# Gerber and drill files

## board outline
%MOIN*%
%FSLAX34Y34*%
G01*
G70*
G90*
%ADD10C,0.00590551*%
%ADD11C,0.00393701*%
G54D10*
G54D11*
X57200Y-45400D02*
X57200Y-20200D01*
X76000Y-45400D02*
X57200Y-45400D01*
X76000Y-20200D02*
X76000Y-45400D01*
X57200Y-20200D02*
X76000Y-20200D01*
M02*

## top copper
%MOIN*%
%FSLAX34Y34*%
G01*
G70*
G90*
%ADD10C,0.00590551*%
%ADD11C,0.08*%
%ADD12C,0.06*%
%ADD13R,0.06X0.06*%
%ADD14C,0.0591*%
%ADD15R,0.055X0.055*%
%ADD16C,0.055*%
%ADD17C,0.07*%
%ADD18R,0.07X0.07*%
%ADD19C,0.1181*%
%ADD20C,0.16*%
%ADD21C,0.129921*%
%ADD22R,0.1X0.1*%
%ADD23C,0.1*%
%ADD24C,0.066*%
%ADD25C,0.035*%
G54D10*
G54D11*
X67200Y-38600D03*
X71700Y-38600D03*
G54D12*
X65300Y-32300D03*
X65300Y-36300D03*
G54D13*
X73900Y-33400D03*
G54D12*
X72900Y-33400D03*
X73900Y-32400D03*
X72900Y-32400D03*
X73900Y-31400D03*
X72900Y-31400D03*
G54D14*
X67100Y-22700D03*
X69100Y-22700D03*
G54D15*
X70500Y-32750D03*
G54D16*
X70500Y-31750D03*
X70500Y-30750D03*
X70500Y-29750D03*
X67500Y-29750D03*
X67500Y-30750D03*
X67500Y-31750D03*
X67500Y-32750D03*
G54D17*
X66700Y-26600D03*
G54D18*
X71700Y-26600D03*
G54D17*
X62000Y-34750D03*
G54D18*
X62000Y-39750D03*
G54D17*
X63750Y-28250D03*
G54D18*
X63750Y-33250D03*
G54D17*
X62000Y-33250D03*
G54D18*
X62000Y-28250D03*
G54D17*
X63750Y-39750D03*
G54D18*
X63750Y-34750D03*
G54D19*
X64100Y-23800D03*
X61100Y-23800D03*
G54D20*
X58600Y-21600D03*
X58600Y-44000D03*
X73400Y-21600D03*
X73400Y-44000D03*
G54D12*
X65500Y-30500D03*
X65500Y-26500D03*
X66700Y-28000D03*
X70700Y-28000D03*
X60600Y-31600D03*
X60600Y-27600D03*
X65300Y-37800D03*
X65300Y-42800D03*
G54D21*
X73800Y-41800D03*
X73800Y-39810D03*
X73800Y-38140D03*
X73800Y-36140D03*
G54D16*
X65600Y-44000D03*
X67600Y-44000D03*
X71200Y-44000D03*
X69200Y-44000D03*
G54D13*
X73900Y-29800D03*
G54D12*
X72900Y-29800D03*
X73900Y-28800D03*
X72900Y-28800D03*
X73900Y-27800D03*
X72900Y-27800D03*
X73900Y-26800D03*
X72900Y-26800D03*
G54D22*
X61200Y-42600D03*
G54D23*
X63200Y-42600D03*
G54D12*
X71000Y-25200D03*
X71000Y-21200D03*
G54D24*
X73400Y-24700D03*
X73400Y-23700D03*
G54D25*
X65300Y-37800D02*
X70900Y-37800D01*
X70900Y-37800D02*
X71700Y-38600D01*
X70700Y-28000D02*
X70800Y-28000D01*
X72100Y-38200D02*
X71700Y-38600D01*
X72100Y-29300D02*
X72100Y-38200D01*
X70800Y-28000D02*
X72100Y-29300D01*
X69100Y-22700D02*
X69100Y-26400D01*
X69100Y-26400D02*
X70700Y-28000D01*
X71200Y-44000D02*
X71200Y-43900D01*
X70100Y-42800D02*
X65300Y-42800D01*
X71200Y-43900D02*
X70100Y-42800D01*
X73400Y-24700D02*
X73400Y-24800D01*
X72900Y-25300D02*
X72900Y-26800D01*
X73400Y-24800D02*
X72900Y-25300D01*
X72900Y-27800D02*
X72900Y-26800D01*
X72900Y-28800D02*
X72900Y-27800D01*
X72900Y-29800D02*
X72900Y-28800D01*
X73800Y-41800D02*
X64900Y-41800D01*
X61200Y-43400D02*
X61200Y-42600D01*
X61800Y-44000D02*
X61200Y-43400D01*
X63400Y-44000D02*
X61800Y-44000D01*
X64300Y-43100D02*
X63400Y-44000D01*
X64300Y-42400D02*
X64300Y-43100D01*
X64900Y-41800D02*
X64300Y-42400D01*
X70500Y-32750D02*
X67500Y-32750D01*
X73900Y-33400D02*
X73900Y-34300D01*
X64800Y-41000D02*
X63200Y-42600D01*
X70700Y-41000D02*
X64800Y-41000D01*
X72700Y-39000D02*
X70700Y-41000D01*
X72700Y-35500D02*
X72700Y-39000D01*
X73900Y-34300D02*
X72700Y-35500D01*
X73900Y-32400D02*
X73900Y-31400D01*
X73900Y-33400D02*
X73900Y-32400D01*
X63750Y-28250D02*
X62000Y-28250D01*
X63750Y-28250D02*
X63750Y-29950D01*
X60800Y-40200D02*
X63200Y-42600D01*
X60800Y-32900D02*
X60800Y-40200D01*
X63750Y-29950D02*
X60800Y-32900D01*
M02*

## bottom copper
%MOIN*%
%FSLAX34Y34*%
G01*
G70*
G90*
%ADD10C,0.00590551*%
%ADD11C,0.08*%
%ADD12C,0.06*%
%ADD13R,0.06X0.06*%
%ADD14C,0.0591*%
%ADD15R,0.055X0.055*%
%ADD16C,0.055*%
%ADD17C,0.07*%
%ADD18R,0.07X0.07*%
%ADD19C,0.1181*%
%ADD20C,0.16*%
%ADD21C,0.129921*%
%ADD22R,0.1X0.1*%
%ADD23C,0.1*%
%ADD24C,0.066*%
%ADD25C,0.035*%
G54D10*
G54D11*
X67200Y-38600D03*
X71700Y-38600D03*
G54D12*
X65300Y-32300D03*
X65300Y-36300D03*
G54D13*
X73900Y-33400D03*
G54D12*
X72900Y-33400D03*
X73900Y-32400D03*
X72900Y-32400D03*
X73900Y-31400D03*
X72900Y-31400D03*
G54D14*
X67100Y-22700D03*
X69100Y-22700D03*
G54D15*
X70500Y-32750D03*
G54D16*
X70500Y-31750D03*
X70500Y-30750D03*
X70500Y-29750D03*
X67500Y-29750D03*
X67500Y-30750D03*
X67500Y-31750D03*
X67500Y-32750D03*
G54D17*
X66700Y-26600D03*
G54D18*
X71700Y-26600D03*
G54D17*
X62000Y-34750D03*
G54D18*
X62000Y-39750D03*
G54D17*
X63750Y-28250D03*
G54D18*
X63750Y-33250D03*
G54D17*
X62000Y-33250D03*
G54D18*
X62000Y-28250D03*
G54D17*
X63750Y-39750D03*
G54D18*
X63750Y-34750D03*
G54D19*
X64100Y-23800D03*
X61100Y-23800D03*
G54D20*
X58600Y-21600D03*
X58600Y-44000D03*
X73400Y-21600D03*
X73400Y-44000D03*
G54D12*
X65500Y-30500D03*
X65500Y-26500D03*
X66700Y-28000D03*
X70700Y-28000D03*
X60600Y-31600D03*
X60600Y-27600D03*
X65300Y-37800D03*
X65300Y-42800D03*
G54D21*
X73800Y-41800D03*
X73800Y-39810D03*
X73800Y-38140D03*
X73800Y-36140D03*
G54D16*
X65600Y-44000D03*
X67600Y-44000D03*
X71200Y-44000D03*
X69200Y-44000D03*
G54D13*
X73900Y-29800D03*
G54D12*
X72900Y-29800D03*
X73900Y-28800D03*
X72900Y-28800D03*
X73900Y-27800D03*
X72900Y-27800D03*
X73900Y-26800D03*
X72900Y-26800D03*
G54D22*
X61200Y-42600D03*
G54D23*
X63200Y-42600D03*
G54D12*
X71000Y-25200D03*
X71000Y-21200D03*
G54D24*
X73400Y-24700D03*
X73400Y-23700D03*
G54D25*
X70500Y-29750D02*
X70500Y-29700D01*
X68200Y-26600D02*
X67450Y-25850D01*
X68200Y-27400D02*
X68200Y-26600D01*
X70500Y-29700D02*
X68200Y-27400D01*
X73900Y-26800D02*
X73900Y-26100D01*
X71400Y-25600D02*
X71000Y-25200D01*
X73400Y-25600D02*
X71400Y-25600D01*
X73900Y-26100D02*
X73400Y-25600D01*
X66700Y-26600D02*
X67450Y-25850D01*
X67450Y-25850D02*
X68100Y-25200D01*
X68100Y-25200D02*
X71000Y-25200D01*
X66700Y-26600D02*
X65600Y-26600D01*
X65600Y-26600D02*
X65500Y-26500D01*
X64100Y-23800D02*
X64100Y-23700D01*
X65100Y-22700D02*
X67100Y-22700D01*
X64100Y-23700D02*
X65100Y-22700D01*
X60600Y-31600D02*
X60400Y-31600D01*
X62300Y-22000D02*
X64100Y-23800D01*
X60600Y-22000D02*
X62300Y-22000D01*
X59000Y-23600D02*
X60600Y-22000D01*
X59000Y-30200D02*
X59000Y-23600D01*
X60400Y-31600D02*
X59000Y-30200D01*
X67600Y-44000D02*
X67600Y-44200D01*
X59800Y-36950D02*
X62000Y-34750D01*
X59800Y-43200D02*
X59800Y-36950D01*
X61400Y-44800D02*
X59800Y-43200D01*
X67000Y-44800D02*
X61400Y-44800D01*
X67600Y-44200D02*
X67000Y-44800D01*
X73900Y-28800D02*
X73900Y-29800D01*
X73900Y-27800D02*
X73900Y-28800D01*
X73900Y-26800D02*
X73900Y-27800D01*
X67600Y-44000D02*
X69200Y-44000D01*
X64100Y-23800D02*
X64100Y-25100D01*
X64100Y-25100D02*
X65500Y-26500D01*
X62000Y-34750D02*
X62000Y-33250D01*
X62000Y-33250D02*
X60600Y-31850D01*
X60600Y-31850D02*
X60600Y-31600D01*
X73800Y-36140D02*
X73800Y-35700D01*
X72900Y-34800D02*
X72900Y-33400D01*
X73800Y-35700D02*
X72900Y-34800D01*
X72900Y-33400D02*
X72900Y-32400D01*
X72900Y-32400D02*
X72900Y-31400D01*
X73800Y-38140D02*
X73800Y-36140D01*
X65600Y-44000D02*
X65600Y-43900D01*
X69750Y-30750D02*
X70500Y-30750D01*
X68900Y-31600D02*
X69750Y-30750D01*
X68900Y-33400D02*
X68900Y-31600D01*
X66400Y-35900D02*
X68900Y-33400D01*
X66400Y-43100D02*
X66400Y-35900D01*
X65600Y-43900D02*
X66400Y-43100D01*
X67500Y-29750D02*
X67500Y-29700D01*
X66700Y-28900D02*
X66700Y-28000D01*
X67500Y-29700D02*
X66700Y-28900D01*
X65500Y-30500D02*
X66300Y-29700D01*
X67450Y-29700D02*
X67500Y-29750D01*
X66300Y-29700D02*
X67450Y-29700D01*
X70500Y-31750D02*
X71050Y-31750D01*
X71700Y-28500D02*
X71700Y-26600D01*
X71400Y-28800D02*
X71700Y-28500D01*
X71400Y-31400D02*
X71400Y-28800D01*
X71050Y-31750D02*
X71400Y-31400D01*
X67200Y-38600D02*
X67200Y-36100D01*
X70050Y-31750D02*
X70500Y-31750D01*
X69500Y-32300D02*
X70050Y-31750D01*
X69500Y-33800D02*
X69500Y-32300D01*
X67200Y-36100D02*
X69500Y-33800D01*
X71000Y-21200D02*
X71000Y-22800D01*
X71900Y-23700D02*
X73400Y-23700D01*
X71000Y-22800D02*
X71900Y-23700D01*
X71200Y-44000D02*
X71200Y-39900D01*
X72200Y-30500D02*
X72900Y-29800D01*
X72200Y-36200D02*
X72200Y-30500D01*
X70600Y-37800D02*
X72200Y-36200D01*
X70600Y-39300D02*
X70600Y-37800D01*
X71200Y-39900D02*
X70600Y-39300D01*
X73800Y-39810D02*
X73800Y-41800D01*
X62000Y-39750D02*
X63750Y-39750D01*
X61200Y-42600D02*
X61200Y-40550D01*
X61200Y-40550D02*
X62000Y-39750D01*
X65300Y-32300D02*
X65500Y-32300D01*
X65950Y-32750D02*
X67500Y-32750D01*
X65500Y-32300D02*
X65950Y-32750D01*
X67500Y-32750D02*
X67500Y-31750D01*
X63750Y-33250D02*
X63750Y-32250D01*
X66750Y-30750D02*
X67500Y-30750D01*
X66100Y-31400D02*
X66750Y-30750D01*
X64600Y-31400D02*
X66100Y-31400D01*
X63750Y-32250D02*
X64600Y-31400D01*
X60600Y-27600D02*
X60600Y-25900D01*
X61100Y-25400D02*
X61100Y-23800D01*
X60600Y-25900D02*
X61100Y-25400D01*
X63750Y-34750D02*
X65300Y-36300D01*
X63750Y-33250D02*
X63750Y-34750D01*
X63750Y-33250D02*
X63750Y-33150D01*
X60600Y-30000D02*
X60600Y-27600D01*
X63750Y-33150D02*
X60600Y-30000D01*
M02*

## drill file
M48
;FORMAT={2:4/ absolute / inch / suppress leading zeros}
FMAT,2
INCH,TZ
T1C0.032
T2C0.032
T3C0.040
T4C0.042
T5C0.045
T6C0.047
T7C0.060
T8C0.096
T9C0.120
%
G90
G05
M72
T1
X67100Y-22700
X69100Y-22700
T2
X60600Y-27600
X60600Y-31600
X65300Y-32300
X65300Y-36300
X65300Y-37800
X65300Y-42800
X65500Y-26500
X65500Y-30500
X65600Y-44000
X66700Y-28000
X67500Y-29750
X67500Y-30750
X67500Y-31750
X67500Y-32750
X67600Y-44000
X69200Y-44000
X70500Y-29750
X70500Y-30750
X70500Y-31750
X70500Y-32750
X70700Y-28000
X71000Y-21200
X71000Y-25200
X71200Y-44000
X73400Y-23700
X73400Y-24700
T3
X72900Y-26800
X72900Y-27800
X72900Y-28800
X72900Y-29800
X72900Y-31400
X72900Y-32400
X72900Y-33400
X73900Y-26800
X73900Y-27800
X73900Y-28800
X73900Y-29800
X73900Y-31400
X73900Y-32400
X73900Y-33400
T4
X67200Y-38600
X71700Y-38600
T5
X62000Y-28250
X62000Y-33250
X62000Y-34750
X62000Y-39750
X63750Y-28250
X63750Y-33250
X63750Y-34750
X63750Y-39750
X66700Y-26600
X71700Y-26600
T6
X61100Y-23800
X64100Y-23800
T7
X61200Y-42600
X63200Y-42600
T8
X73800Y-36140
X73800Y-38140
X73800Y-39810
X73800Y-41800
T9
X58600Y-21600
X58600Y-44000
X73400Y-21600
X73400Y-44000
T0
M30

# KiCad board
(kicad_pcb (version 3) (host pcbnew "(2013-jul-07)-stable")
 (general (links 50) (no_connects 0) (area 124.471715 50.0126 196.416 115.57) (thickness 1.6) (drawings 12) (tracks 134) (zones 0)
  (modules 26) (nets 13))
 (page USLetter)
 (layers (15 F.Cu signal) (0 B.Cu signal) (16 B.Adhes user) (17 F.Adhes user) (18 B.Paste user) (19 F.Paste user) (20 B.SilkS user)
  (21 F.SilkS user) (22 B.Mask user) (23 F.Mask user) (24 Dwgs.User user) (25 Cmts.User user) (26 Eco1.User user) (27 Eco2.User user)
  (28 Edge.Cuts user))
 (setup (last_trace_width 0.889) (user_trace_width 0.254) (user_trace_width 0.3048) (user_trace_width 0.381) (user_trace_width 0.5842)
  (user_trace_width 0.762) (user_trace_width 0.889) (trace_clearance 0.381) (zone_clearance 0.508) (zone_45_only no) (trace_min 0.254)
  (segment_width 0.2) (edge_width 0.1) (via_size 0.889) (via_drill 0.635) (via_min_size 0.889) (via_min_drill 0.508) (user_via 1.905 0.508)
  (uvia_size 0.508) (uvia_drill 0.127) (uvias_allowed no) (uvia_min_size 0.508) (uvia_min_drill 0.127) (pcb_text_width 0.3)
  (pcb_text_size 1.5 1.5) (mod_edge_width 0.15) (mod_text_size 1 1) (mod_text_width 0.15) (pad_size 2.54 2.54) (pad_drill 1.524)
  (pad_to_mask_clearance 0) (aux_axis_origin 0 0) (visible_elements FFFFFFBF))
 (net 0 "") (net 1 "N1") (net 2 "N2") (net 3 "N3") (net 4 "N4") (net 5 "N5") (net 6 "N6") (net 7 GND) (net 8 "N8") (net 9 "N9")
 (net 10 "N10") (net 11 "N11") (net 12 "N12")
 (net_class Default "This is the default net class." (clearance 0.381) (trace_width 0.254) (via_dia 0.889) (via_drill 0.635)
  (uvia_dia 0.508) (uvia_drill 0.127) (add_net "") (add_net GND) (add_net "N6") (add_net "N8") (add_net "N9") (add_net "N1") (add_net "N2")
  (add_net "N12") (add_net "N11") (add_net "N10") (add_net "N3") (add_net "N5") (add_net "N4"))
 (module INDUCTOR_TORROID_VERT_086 (layer F.Cu) (at 176.276 98.044 90)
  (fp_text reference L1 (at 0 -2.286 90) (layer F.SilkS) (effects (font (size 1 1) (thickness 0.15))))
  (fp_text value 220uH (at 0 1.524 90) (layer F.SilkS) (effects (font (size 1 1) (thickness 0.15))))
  (pad 1 thru_hole circle (at 0 -5.588 90) (size 2.032 2.032) (drill 1.0668) (layers *.Cu *.Mask F.SilkS) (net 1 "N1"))
  (pad 2 thru_hole circle (at 0 5.842 90) (size 2.032 2.032) (drill 1.0668) (layers *.Cu *.Mask F.SilkS) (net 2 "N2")))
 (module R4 (layer F.Cu) (at 165.862 87.122 270) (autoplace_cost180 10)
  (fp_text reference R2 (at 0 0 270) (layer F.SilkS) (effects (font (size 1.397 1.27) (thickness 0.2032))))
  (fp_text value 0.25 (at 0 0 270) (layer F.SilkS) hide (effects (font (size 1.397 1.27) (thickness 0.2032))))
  (pad 1 thru_hole circle (at -5.08 0 270) (size 1.524 1.524) (drill 0.8128) (layers *.Cu *.Mask F.SilkS) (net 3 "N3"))
  (pad 2 thru_hole circle (at 5.08 0 270) (size 1.524 1.524) (drill 0.8128) (layers *.Cu *.Mask F.SilkS) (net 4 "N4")))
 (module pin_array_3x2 (layer F.Cu) (at 186.436 82.296 90)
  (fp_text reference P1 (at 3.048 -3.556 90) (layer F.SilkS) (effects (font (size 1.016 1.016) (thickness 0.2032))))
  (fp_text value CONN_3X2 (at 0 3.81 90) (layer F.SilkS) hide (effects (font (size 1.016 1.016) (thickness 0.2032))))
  (pad 1 thru_hole rect (at -2.54 1.27 90) (size 1.524 1.524) (drill 1.016) (layers *.Cu *.Mask F.SilkS) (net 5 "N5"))
  (pad 2 thru_hole circle (at -2.54 -1.27 90) (size 1.524 1.524) (drill 1.016) (layers *.Cu *.Mask F.SilkS) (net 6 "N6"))
  (pad 3 thru_hole circle (at 0 1.27 90) (size 1.524 1.524) (drill 1.016) (layers *.Cu *.Mask F.SilkS) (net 5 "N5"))
  (pad 4 thru_hole circle (at 0 -1.27 90) (size 1.524 1.524) (drill 1.016) (layers *.Cu *.Mask F.SilkS) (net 6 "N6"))
  (pad 5 thru_hole circle (at 2.54 1.27 90) (size 1.524 1.524) (drill 1.016) (layers *.Cu *.Mask F.SilkS) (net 5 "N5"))
  (pad 6 thru_hole circle (at 2.54 -1.27 90) (size 1.524 1.524) (drill 1.016) (layers *.Cu *.Mask F.SilkS) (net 6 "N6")))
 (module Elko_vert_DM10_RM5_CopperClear (layer F.Cu) (at 172.974 57.658 180)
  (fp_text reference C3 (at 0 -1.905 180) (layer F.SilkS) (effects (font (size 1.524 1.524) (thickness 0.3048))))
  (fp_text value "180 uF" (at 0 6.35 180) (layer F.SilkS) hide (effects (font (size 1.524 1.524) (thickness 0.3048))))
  (pad 2 thru_hole circle (at 2.54 0 180) (size 1.50114 1.50114) (drill 0.8001) (layers *.Cu *.Mask F.SilkS) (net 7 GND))
  (pad 1 thru_hole circle (at -2.54 0 180) (size 1.50114 1.50114) (drill 0.8001) (layers *.Cu *.Mask F.SilkS) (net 2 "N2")))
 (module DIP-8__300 (layer F.Cu) (at 175.26 79.375 90)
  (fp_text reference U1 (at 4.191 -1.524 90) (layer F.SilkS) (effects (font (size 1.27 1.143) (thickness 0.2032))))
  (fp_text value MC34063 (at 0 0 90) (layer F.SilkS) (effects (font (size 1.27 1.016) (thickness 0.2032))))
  (pad 1 thru_hole rect (at -3.81 3.81 90) (size 1.397 1.397) (drill 0.8128) (layers *.Cu *.Mask F.SilkS) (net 3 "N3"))
  (pad 2 thru_hole circle (at -1.27 3.81 90) (size 1.397 1.397) (drill 0.8128) (layers *.Cu *.Mask F.SilkS) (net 1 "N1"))
  (pad 3 thru_hole circle (at 1.27 3.81 90) (size 1.397 1.397) (drill 0.8128) (layers *.Cu *.Mask F.SilkS) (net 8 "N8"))
  (pad 4 thru_hole circle (at 3.81 3.81 90) (size 1.397 1.397) (drill 0.8128) (layers *.Cu *.Mask F.SilkS) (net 7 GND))
  (pad 5 thru_hole circle (at 3.81 -3.81 90) (size 1.397 1.397) (drill 0.8128) (layers *.Cu *.Mask F.SilkS) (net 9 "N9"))
  (pad 6 thru_hole circle (at 1.27 -3.81 90) (size 1.397 1.397) (drill 0.8128) (layers *.Cu *.Mask F.SilkS) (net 4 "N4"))
  (pad 7 thru_hole circle (at -1.27 -3.81 90) (size 1.397 1.397) (drill 0.8128) (layers *.Cu *.Mask F.SilkS) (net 3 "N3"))
  (pad 8 thru_hole circle (at -3.81 -3.81 90) (size 1.397 1.397) (drill 0.8128) (layers *.Cu *.Mask F.SilkS) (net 3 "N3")))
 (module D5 (layer F.Cu) (at 175.768 67.564)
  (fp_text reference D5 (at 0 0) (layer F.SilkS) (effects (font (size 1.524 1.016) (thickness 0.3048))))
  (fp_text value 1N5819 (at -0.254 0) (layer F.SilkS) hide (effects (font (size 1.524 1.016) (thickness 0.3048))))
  (pad 1 thru_hole circle (at -6.35 0) (size 1.778 1.778) (drill 1.143) (layers *.Cu *.Mask F.SilkS) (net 7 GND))
  (pad 2 thru_hole rect (at 6.35 0) (size 1.778 1.778) (drill 1.143) (layers *.Cu *.Mask F.SilkS) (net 1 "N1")))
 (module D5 (layer F.Cu) (at 157.48 94.615 270)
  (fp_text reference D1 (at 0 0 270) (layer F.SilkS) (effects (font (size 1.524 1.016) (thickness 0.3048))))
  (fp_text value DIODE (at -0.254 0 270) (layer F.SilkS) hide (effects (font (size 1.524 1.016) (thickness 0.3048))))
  (pad 1 thru_hole circle (at -6.35 0 270) (size 1.778 1.778) (drill 1.143) (layers *.Cu *.Mask F.SilkS) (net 7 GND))
  (pad 2 thru_hole rect (at 6.35 0 270) (size 1.778 1.778) (drill 1.143) (layers *.Cu *.Mask F.SilkS) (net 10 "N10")))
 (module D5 (layer F.Cu) (at 161.925 78.105 270)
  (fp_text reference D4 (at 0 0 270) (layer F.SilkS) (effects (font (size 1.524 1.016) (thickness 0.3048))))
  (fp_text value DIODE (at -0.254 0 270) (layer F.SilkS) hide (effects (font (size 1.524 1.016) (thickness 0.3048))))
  (pad 1 thru_hole circle (at -6.35 0 270) (size 1.778 1.778) (drill 1.143) (layers *.Cu *.Mask F.SilkS) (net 5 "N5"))
  (pad 2 thru_hole rect (at 6.35 0 270) (size 1.778 1.778) (drill 1.143) (layers *.Cu *.Mask F.SilkS) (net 4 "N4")))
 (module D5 (layer F.Cu) (at 157.48 78.105 90)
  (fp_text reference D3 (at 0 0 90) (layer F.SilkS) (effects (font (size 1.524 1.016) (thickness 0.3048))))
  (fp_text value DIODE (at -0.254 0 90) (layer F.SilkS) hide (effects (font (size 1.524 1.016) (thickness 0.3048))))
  (pad 1 thru_hole circle (at -6.35 0 90) (size 1.778 1.778) (drill 1.143) (layers *.Cu *.Mask F.SilkS) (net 7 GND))
  (pad 2 thru_hole rect (at 6.35 0 90) (size 1.778 1.778) (drill 1.143) (layers *.Cu *.Mask F.SilkS) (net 5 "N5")))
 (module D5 (layer F.Cu) (at 161.925 94.615 90)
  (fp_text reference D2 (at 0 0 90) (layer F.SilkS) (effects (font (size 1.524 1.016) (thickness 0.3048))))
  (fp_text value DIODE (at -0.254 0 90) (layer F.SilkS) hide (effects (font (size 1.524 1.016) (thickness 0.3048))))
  (pad 1 thru_hole circle (at -6.35 0 90) (size 1.778 1.778) (drill 1.143) (layers *.Cu *.Mask F.SilkS) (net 10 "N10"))
  (pad 2 thru_hole rect (at 6.35 0 90) (size 1.778 1.778) (drill 1.143) (layers *.Cu *.Mask F.SilkS) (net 4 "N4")))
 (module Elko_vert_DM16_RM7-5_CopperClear (layer F.Cu) (at 159.004 60.452)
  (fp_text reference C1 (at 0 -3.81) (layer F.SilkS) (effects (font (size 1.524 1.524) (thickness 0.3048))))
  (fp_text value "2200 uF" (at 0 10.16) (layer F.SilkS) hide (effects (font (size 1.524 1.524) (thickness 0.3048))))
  (pad 2 thru_hole circle (at 3.81 0) (size 2.99974 2.99974) (drill 1.19888) (layers *.Cu *.Mask F.SilkS) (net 7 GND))
  (pad 1 thru_hole circle (at -3.81 0) (size 2.99974 2.99974) (drill 1.19888) (layers *.Cu *.Mask F.SilkS) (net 4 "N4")))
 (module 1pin (layer F.Cu) (at 148.844 54.864)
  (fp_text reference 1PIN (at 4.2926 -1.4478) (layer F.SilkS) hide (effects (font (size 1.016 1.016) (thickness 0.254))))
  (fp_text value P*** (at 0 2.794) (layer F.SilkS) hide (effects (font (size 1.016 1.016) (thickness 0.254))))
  (pad 1 thru_hole circle (at 0 0) (size 4.064 4.064) (drill 3.048) (layers *.Cu *.Mask F.SilkS)))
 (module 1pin (layer F.Cu) (at 148.844 111.76)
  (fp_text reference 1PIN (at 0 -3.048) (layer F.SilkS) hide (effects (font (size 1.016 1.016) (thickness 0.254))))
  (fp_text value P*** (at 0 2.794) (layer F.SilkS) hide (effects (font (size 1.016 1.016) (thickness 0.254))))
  (pad 1 thru_hole circle (at 0 0) (size 4.064 4.064) (drill 3.048) (layers *.Cu *.Mask F.SilkS)))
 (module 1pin (layer F.Cu) (at 186.436 54.864)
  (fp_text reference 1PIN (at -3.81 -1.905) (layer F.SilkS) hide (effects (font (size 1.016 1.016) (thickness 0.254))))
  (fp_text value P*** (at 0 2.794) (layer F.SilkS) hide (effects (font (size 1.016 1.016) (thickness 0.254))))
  (pad 1 thru_hole circle (at 0 0) (size 4.064 4.064) (drill 3.048) (layers *.Cu *.Mask F.SilkS)))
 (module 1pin (layer F.Cu) (at 186.436 111.76)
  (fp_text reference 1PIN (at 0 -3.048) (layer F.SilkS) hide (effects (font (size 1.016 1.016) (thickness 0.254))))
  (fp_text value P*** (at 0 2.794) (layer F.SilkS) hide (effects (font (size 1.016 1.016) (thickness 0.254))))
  (pad 1 thru_hole circle (at 0 0) (size 4.064 4.064) (drill 3.048) (layers *.Cu *.Mask F.SilkS)))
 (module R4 (layer F.Cu) (at 166.37 72.39 90) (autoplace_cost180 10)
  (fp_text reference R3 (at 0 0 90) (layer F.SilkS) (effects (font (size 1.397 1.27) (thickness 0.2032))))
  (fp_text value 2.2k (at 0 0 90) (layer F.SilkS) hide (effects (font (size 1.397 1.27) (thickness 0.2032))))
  (pad 1 thru_hole circle (at -5.08 0 90) (size 1.524 1.524) (drill 0.8128) (layers *.Cu *.Mask F.SilkS) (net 9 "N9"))
  (pad 2 thru_hole circle (at 5.08 0 90) (size 1.524 1.524) (drill 0.8128) (layers *.Cu *.Mask F.SilkS) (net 7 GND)))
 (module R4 (layer F.Cu) (at 174.498 71.12) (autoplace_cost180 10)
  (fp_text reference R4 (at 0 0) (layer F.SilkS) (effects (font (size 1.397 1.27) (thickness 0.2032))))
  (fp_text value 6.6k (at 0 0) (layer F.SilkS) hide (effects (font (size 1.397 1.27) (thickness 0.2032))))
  (pad 1 thru_hole circle (at -5.08 0) (size 1.524 1.524) (drill 0.8128) (layers *.Cu *.Mask F.SilkS) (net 9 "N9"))
  (pad 2 thru_hole circle (at 5.08 0) (size 1.524 1.524) (drill 0.8128) (layers *.Cu *.Mask F.SilkS) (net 2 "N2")))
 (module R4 (layer F.Cu) (at 153.924 75.184 90) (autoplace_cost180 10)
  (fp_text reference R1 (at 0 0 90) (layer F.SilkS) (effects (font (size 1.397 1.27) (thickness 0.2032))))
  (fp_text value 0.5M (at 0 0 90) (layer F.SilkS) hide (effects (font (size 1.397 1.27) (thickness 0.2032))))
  (pad 1 thru_hole circle (at -5.08 0 90) (size 1.524 1.524) (drill 0.8128) (layers *.Cu *.Mask F.SilkS) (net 7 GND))
  (pad 2 thru_hole circle (at 5.08 0 90) (size 1.524 1.524) (drill 0.8128) (layers *.Cu *.Mask F.SilkS) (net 4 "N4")))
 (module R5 (layer F.Cu) (at 165.862 102.362 270) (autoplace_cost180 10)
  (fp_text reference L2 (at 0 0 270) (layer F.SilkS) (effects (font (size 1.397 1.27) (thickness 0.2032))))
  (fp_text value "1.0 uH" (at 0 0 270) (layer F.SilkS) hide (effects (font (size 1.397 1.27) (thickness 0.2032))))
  (pad 1 thru_hole circle (at -6.35 0 270) (size 1.524 1.524) (drill 0.8128) (layers *.Cu *.Mask F.SilkS) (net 2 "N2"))
  (pad 2 thru_hole circle (at 6.35 0 270) (size 1.524 1.524) (drill 0.8128) (layers *.Cu *.Mask F.SilkS) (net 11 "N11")))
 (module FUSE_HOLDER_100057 (layer F.Cu) (at 187.452 98.552 90)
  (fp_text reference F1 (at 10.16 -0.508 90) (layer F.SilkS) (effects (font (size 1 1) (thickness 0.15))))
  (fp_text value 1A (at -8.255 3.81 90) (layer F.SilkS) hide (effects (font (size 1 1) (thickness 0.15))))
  (pad 1 thru_hole circle (at -7.62 0 90) (size 3.3 3.3) (drill 2.44) (layers *.Cu *.Mask F.SilkS) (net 10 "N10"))
  (pad 1 thru_hole circle (at -2.5654 0 90) (size 3.3 3.3) (drill 2.44) (layers *.Cu *.Mask F.SilkS) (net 10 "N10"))
  (pad 2 thru_hole circle (at 1.6764 0 90) (size 3.3 3.3) (drill 2.44) (layers *.Cu *.Mask F.SilkS) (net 6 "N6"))
  (pad 2 thru_hole circle (at 6.7564 0 90) (size 3.3 3.3) (drill 2.44) (layers *.Cu *.Mask F.SilkS) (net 6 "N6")))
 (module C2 (layer F.Cu) (at 169.164 111.76)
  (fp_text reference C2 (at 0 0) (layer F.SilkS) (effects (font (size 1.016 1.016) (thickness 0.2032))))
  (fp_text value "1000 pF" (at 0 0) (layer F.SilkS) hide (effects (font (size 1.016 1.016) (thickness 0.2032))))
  (pad 1 thru_hole circle (at -2.54 0) (size 1.397 1.397) (drill 0.8128) (layers *.Cu *.Mask F.SilkS) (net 8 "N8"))
  (pad 2 thru_hole circle (at 2.54 0) (size 1.397 1.397) (drill 0.8128) (layers *.Cu *.Mask F.SilkS) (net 7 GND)))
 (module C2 (layer F.Cu) (at 178.308 111.76 180)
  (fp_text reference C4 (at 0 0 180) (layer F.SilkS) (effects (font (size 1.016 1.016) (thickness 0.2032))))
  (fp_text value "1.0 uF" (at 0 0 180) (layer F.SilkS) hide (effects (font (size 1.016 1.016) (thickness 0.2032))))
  (pad 1 thru_hole circle (at -2.54 0 180) (size 1.397 1.397) (drill 0.8128) (layers *.Cu *.Mask F.SilkS) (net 11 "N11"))
  (pad 2 thru_hole circle (at 2.54 0 180) (size 1.397 1.397) (drill 0.8128) (layers *.Cu *.Mask F.SilkS) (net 7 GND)))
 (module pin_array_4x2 (layer F.Cu) (at 186.436 71.882 90)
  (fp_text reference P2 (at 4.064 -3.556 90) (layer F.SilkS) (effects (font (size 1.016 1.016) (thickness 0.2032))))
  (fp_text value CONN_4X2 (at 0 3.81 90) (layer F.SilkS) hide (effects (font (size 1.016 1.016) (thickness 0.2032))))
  (pad 1 thru_hole rect (at -3.81 1.27 90) (size 1.524 1.524) (drill 1.016) (layers *.Cu *.Mask F.SilkS) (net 7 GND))
  (pad 2 thru_hole circle (at -3.81 -1.27 90) (size 1.524 1.524) (drill 1.016) (layers *.Cu *.Mask F.SilkS) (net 11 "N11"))
  (pad 3 thru_hole circle (at -1.27 1.27 90) (size 1.524 1.524) (drill 1.016) (layers *.Cu *.Mask F.SilkS) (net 7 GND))
  (pad 4 thru_hole circle (at -1.27 -1.27 90) (size 1.524 1.524) (drill 1.016) (layers *.Cu *.Mask F.SilkS) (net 11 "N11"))
  (pad 5 thru_hole circle (at 1.27 1.27 90) (size 1.524 1.524) (drill 1.016) (layers *.Cu *.Mask F.SilkS) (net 7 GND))
  (pad 6 thru_hole circle (at 1.27 -1.27 90) (size 1.524 1.524) (drill 1.016) (layers *.Cu *.Mask F.SilkS) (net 11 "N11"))
  (pad 7 thru_hole circle (at 3.81 1.27 90) (size 1.524 1.524) (drill 1.016) (layers *.Cu *.Mask F.SilkS) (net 7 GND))
  (pad 8 thru_hole circle (at 3.81 -1.27 90) (size 1.524 1.524) (drill 1.016) (layers *.Cu *.Mask F.SilkS) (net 11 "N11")))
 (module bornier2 (layer F.Cu) (at 157.988 108.204)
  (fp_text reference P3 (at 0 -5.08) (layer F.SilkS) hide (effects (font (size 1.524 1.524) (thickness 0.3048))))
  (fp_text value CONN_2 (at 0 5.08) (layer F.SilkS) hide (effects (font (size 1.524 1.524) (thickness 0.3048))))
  (pad 1 thru_hole rect (at -2.54 0) (size 2.54 2.54) (drill 1.524) (layers *.Cu *.Mask F.SilkS) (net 10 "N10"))
  (pad 2 thru_hole circle (at 2.54 0) (size 2.54 2.54) (drill 1.524) (layers *.Cu *.Mask F.SilkS) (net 5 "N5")))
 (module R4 (layer F.Cu) (at 180.34 58.928 90) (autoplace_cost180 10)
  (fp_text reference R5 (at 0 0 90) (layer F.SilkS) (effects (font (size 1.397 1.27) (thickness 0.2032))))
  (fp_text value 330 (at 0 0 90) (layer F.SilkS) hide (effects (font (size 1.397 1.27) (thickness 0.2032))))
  (pad 1 thru_hole circle (at -5.08 0 90) (size 1.524 1.524) (drill 0.8128) (layers *.Cu *.Mask F.SilkS) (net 7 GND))
  (pad 2 thru_hole circle (at 5.08 0 90) (size 1.524 1.524) (drill 0.8128) (layers *.Cu *.Mask F.SilkS) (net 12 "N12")))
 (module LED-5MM (layer F.Cu) (at 186.436 61.468 90)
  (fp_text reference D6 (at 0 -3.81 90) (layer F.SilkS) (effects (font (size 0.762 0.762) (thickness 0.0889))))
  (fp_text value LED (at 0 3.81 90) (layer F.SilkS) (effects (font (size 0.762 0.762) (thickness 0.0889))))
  (pad 1 thru_hole circle (at -1.27 0 90) (size 1.6764 1.6764) (drill 0.8128) (layers *.Cu *.Mask F.SilkS) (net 11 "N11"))
  (pad 2 thru_hole circle (at 1.27 0 90) (size 1.6764 1.6764) (drill 0.8128) (layers *.Cu *.Mask F.SilkS) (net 12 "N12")))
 (gr_line (start 145.288 115.316) (end 145.288 51.308) (angle 90) (layer Edge.Cuts) (width 0.1))
 (gr_line (start 193.04 115.316) (end 145.288 115.316) (angle 90) (layer Edge.Cuts) (width 0.1))
 (gr_line (start 193.04 51.308) (end 193.04 115.316) (angle 90) (layer Edge.Cuts) (width 0.1))
 (gr_line (start 145.288 51.308) (end 193.04 51.308) (angle 90) (layer Edge.Cuts) (width 0.1))
 (segment (start 179.07 75.565) (end 179.07 75.438) (width 0.889) (layer B.Cu) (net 7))
 (segment (start 173.228 67.564) (end 171.323 65.659) (width 0.889) (layer B.Cu) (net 7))
 (segment (start 173.228 69.596) (end 173.228 67.564) (width 0.889) (layer B.Cu) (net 7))
 (segment (start 179.07 75.438) (end 173.228 69.596) (width 0.889) (layer B.Cu) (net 7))
 (segment (start 187.706 68.072) (end 187.706 66.294) (width 0.889) (layer B.Cu) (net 7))
 (segment (start 181.356 65.024) (end 180.34 64.008) (width 0.889) (layer B.Cu) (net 7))
 (segment (start 186.436 65.024) (end 181.356 65.024) (width 0.889) (layer B.Cu) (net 7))
 (segment (start 187.706 66.294) (end 186.436 65.024) (width 0.889) (layer B.Cu) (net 7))
 (segment (start 169.418 67.564) (end 171.323 65.659) (width 0.889) (layer B.Cu) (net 7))
 (segment (start 171.323 65.659) (end 172.974 64.008) (width 0.889) (layer B.Cu) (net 7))
 (segment (start 172.974 64.008) (end 180.34 64.008) (width 0.889) (layer B.Cu) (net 7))
 (segment (start 169.418 67.564) (end 166.624 67.564) (width 0.889) (layer B.Cu) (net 7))
 (segment (start 166.624 67.564) (end 166.37 67.31) (width 0.889) (layer B.Cu) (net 7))
 (segment (start 162.814 60.452) (end 162.814 60.198) (width 0.889) (layer B.Cu) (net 7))
 (segment (start 165.354 57.658) (end 170.434 57.658) (width 0.889) (layer B.Cu) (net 7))
 (segment (start 162.814 60.198) (end 165.354 57.658) (width 0.889) (layer B.Cu) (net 7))
 (segment (start 153.924 80.264) (end 153.416 80.264) (width 0.889) (layer B.Cu) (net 7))
 (segment (start 158.242 55.88) (end 162.814 60.452) (width 0.889) (layer B.Cu) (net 7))
 (segment (start 153.924 55.88) (end 158.242 55.88) (width 0.889) (layer B.Cu) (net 7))
 (segment (start 149.86 59.944) (end 153.924 55.88) (width 0.889) (layer B.Cu) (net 7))
 (segment (start 149.86 76.708) (end 149.86 59.944) (width 0.889) (layer B.Cu) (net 7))
 (segment (start 153.416 80.264) (end 149.86 76.708) (width 0.889) (layer B.Cu) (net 7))
 (segment (start 171.704 111.76) (end 171.704 112.268) (width 0.889) (layer B.Cu) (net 7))
 (segment (start 151.892 93.853) (end 157.48 88.265) (width 0.889) (layer B.Cu) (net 7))
 (segment (start 151.892 109.728) (end 151.892 93.853) (width 0.889) (layer B.Cu) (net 7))
 (segment (start 155.956 113.792) (end 151.892 109.728) (width 0.889) (layer B.Cu) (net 7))
 (segment (start 170.18 113.792) (end 155.956 113.792) (width 0.889) (layer B.Cu) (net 7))
 (segment (start 171.704 112.268) (end 170.18 113.792) (width 0.889) (layer B.Cu) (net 7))
 (segment (start 187.706 73.152) (end 187.706 75.692) (width 0.889) (layer B.Cu) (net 7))
 (segment (start 187.706 70.612) (end 187.706 73.152) (width 0.889) (layer B.Cu) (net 7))
 (segment (start 187.706 68.072) (end 187.706 70.612) (width 0.889) (layer B.Cu) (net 7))
 (segment (start 171.704 111.76) (end 175.768 111.76) (width 0.889) (layer B.Cu) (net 7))
 (segment (start 162.814 60.452) (end 162.814 63.754) (width 0.889) (layer B.Cu) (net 7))
 (segment (start 162.814 63.754) (end 166.37 67.31) (width 0.889) (layer B.Cu) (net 7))
 (segment (start 157.48 88.265) (end 157.48 84.455) (width 0.889) (layer B.Cu) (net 7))
 (segment (start 157.48 84.455) (end 153.924 80.899) (width 0.889) (layer B.Cu) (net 7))
 (segment (start 153.924 80.899) (end 153.924 80.264) (width 0.889) (layer B.Cu) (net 7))
 (segment (start 187.452 91.7956) (end 187.452 90.678) (width 0.889) (layer B.Cu) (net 6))
 (segment (start 185.166 88.392) (end 185.166 84.836) (width 0.889) (layer B.Cu) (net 6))
 (segment (start 187.452 90.678) (end 185.166 88.392) (width 0.889) (layer B.Cu) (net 6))
 (segment (start 185.166 84.836) (end 185.166 82.296) (width 0.889) (layer B.Cu) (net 6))
 (segment (start 185.166 82.296) (end 185.166 79.756) (width 0.889) (layer B.Cu) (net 6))
 (segment (start 187.452 96.8756) (end 187.452 91.7956) (width 0.889) (layer B.Cu) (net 6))
 (segment (start 166.624 111.76) (end 166.624 111.506) (width 0.889) (layer B.Cu) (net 8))
 (segment (start 177.165 78.105) (end 179.07 78.105) (width 0.889) (layer B.Cu) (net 8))
 (segment (start 175.006 80.264) (end 177.165 78.105) (width 0.889) (layer B.Cu) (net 8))
 (segment (start 175.006 84.836) (end 175.006 80.264) (width 0.889) (layer B.Cu) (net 8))
 (segment (start 168.656 91.186) (end 175.006 84.836) (width 0.889) (layer B.Cu) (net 8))
 (segment (start 168.656 109.474) (end 168.656 91.186) (width 0.889) (layer B.Cu) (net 8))
 (segment (start 166.624 111.506) (end 168.656 109.474) (width 0.889) (layer B.Cu) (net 8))
 (segment (start 171.45 75.565) (end 171.45 75.438) (width 0.889) (layer B.Cu) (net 9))
 (segment (start 169.418 73.406) (end 169.418 71.12) (width 0.889) (layer B.Cu) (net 9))
 (segment (start 171.45 75.438) (end 169.418 73.406) (width 0.889) (layer B.Cu) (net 9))
 (segment (start 166.37 77.47) (end 168.402 75.438) (width 0.889) (layer B.Cu) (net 9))
 (segment (start 171.323 75.438) (end 171.45 75.565) (width 0.889) (layer B.Cu) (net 9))
 (segment (start 168.402 75.438) (end 171.323 75.438) (width 0.889) (layer B.Cu) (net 9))
 (segment (start 179.07 80.645) (end 180.467 80.645) (width 0.889) (layer B.Cu) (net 1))
 (segment (start 182.118 72.39) (end 182.118 67.564) (width 0.889) (layer B.Cu) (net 1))
 (segment (start 181.356 73.152) (end 182.118 72.39) (width 0.889) (layer B.Cu) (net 1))
 (segment (start 181.356 79.756) (end 181.356 73.152) (width 0.889) (layer B.Cu) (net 1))
 (segment (start 180.467 80.645) (end 181.356 79.756) (width 0.889) (layer B.Cu) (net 1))
 (segment (start 170.688 98.044) (end 170.688 91.694) (width 0.889) (layer B.Cu) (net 1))
 (segment (start 177.927 80.645) (end 179.07 80.645) (width 0.889) (layer B.Cu) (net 1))
 (segment (start 176.53 82.042) (end 177.927 80.645) (width 0.889) (layer B.Cu) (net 1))
 (segment (start 176.53 85.852) (end 176.53 82.042) (width 0.889) (layer B.Cu) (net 1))
 (segment (start 170.688 91.694) (end 176.53 85.852) (width 0.889) (layer B.Cu) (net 1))
 (segment (start 165.862 96.012) (end 180.086 96.012) (width 0.889) (layer F.Cu) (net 2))
 (segment (start 180.086 96.012) (end 182.118 98.044) (width 0.889) (layer F.Cu) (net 2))
 (segment (start 179.578 71.12) (end 179.832 71.12) (width 0.889) (layer F.Cu) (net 2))
 (segment (start 183.134 97.028) (end 182.118 98.044) (width 0.889) (layer F.Cu) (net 2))
 (segment (start 183.134 74.422) (end 183.134 97.028) (width 0.889) (layer F.Cu) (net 2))
 (segment (start 179.832 71.12) (end 183.134 74.422) (width 0.889) (layer F.Cu) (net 2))
 (segment (start 175.514 57.658) (end 175.514 67.056) (width 0.889) (layer F.Cu) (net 2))
 (segment (start 175.514 67.056) (end 179.578 71.12) (width 0.889) (layer F.Cu) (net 2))
 (segment (start 180.34 53.848) (end 180.34 57.912) (width 0.889) (layer B.Cu) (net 12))
 (segment (start 182.626 60.198) (end 186.436 60.198) (width 0.889) (layer B.Cu) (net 12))
 (segment (start 180.34 57.912) (end 182.626 60.198) (width 0.889) (layer B.Cu) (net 12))
 (segment (start 180.848 111.76) (end 180.848 111.506) (width 0.889) (layer F.Cu) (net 11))
 (segment (start 178.054 108.712) (end 165.862 108.712) (width 0.889) (layer F.Cu) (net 11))
 (segment (start 180.848 111.506) (end 178.054 108.712) (width 0.889) (layer F.Cu) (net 11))
 (segment (start 180.848 111.76) (end 180.848 101.346) (width 0.889) (layer B.Cu) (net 11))
 (segment (start 183.388 77.47) (end 185.166 75.692) (width 0.889) (layer B.Cu) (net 11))
 (segment (start 183.388 91.948) (end 183.388 77.47) (width 0.889) (layer B.Cu) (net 11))
 (segment (start 179.324 96.012) (end 183.388 91.948) (width 0.889) (layer B.Cu) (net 11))
 (segment (start 179.324 99.822) (end 179.324 96.012) (width 0.889) (layer B.Cu) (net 11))
 (segment (start 180.848 101.346) (end 179.324 99.822) (width 0.889) (layer B.Cu) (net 11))
 (segment (start 186.436 62.738) (end 186.436 62.992) (width 0.889) (layer F.Cu) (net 11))
 (segment (start 185.166 64.262) (end 185.166 68.072) (width 0.889) (layer F.Cu) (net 11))
 (segment (start 186.436 62.992) (end 185.166 64.262) (width 0.889) (layer F.Cu) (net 11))
 (segment (start 185.166 70.612) (end 185.166 68.072) (width 0.889) (layer F.Cu) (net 11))
 (segment (start 185.166 73.152) (end 185.166 70.612) (width 0.889) (layer F.Cu) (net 11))
 (segment (start 185.166 75.692) (end 185.166 73.152) (width 0.889) (layer F.Cu) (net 11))
 (segment (start 187.452 106.172) (end 164.846 106.172) (width 0.889) (layer F.Cu) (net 10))
 (segment (start 155.448 110.236) (end 155.448 108.204) (width 0.889) (layer F.Cu) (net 10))
 (segment (start 156.972 111.76) (end 155.448 110.236) (width 0.889) (layer F.Cu) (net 10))
 (segment (start 161.036 111.76) (end 156.972 111.76) (width 0.889) (layer F.Cu) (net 10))
 (segment (start 163.322 109.474) (end 161.036 111.76) (width 0.889) (layer F.Cu) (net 10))
 (segment (start 163.322 107.696) (end 163.322 109.474) (width 0.889) (layer F.Cu) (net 10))
 (segment (start 164.846 106.172) (end 163.322 107.696) (width 0.889) (layer F.Cu) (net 10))
 (segment (start 187.452 101.1174) (end 187.452 106.172) (width 0.889) (layer B.Cu) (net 10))
 (segment (start 157.48 100.965) (end 161.925 100.965) (width 0.889) (layer B.Cu) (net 10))
 (segment (start 155.448 108.204) (end 155.448 102.997) (width 0.889) (layer B.Cu) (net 10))
 (segment (start 155.448 102.997) (end 157.48 100.965) (width 0.889) (layer B.Cu) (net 10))
 (segment (start 165.862 82.042) (end 166.37 82.042) (width 0.889) (layer B.Cu) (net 3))
 (segment (start 167.513 83.185) (end 171.45 83.185) (width 0.889) (layer B.Cu) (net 3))
 (segment (start 166.37 82.042) (end 167.513 83.185) (width 0.889) (layer B.Cu) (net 3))
 (segment (start 171.45 83.185) (end 171.45 80.645) (width 0.889) (layer B.Cu) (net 3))
 (segment (start 179.07 83.185) (end 171.45 83.185) (width 0.889) (layer F.Cu) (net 3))
 (segment (start 187.706 84.836) (end 187.706 87.122) (width 0.889) (layer F.Cu) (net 5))
 (segment (start 164.592 104.14) (end 160.528 108.204) (width 0.889) (layer F.Cu) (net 5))
 (segment (start 179.578 104.14) (end 164.592 104.14) (width 0.889) (layer F.Cu) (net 5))
 (segment (start 184.658 99.06) (end 179.578 104.14) (width 0.889) (layer F.Cu) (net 5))
 (segment (start 184.658 90.17) (end 184.658 99.06) (width 0.889) (layer F.Cu) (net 5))
 (segment (start 187.706 87.122) (end 184.658 90.17) (width 0.889) (layer F.Cu) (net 5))
 (segment (start 187.706 82.296) (end 187.706 79.756) (width 0.889) (layer F.Cu) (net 5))
 (segment (start 187.706 84.836) (end 187.706 82.296) (width 0.889) (layer F.Cu) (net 5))
 (segment (start 161.925 71.755) (end 157.48 71.755) (width 0.889) (layer F.Cu) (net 5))
 (segment (start 161.925 71.755) (end 161.925 76.073) (width 0.889) (layer F.Cu) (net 5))
 (segment (start 154.432 102.108) (end 160.528 108.204) (width 0.889) (layer F.Cu) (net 5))
 (segment (start 154.432 83.566) (end 154.432 102.108) (width 0.889) (layer F.Cu) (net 5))
 (segment (start 161.925 76.073) (end 154.432 83.566) (width 0.889) (layer F.Cu) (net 5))
 (segment (start 161.925 84.455) (end 161.925 81.915) (width 0.889) (layer B.Cu) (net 4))
 (segment (start 169.545 78.105) (end 171.45 78.105) (width 0.889) (layer B.Cu) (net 4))
 (segment (start 167.894 79.756) (end 169.545 78.105) (width 0.889) (layer B.Cu) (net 4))
 (segment (start 164.084 79.756) (end 167.894 79.756) (width 0.889) (layer B.Cu) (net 4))
 (segment (start 161.925 81.915) (end 164.084 79.756) (width 0.889) (layer B.Cu) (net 4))
 (segment (start 153.924 70.104) (end 153.924 65.786) (width 0.889) (layer B.Cu) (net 4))
 (segment (start 155.194 64.516) (end 155.194 60.452) (width 0.889) (layer B.Cu) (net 4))
 (segment (start 153.924 65.786) (end 155.194 64.516) (width 0.889) (layer B.Cu) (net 4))
 (segment (start 161.925 88.265) (end 165.862 92.202) (width 0.889) (layer B.Cu) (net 4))
 (segment (start 161.925 84.455) (end 161.925 88.265) (width 0.889) (layer B.Cu) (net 4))
 (segment (start 161.925 84.455) (end 161.925 84.201) (width 0.889) (layer B.Cu) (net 4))
 (segment (start 153.924 76.2) (end 153.924 70.104) (width 0.889) (layer B.Cu) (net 4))
 (segment (start 161.925 84.201) (end 153.924 76.2) (width 0.889) (layer B.Cu) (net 4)))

